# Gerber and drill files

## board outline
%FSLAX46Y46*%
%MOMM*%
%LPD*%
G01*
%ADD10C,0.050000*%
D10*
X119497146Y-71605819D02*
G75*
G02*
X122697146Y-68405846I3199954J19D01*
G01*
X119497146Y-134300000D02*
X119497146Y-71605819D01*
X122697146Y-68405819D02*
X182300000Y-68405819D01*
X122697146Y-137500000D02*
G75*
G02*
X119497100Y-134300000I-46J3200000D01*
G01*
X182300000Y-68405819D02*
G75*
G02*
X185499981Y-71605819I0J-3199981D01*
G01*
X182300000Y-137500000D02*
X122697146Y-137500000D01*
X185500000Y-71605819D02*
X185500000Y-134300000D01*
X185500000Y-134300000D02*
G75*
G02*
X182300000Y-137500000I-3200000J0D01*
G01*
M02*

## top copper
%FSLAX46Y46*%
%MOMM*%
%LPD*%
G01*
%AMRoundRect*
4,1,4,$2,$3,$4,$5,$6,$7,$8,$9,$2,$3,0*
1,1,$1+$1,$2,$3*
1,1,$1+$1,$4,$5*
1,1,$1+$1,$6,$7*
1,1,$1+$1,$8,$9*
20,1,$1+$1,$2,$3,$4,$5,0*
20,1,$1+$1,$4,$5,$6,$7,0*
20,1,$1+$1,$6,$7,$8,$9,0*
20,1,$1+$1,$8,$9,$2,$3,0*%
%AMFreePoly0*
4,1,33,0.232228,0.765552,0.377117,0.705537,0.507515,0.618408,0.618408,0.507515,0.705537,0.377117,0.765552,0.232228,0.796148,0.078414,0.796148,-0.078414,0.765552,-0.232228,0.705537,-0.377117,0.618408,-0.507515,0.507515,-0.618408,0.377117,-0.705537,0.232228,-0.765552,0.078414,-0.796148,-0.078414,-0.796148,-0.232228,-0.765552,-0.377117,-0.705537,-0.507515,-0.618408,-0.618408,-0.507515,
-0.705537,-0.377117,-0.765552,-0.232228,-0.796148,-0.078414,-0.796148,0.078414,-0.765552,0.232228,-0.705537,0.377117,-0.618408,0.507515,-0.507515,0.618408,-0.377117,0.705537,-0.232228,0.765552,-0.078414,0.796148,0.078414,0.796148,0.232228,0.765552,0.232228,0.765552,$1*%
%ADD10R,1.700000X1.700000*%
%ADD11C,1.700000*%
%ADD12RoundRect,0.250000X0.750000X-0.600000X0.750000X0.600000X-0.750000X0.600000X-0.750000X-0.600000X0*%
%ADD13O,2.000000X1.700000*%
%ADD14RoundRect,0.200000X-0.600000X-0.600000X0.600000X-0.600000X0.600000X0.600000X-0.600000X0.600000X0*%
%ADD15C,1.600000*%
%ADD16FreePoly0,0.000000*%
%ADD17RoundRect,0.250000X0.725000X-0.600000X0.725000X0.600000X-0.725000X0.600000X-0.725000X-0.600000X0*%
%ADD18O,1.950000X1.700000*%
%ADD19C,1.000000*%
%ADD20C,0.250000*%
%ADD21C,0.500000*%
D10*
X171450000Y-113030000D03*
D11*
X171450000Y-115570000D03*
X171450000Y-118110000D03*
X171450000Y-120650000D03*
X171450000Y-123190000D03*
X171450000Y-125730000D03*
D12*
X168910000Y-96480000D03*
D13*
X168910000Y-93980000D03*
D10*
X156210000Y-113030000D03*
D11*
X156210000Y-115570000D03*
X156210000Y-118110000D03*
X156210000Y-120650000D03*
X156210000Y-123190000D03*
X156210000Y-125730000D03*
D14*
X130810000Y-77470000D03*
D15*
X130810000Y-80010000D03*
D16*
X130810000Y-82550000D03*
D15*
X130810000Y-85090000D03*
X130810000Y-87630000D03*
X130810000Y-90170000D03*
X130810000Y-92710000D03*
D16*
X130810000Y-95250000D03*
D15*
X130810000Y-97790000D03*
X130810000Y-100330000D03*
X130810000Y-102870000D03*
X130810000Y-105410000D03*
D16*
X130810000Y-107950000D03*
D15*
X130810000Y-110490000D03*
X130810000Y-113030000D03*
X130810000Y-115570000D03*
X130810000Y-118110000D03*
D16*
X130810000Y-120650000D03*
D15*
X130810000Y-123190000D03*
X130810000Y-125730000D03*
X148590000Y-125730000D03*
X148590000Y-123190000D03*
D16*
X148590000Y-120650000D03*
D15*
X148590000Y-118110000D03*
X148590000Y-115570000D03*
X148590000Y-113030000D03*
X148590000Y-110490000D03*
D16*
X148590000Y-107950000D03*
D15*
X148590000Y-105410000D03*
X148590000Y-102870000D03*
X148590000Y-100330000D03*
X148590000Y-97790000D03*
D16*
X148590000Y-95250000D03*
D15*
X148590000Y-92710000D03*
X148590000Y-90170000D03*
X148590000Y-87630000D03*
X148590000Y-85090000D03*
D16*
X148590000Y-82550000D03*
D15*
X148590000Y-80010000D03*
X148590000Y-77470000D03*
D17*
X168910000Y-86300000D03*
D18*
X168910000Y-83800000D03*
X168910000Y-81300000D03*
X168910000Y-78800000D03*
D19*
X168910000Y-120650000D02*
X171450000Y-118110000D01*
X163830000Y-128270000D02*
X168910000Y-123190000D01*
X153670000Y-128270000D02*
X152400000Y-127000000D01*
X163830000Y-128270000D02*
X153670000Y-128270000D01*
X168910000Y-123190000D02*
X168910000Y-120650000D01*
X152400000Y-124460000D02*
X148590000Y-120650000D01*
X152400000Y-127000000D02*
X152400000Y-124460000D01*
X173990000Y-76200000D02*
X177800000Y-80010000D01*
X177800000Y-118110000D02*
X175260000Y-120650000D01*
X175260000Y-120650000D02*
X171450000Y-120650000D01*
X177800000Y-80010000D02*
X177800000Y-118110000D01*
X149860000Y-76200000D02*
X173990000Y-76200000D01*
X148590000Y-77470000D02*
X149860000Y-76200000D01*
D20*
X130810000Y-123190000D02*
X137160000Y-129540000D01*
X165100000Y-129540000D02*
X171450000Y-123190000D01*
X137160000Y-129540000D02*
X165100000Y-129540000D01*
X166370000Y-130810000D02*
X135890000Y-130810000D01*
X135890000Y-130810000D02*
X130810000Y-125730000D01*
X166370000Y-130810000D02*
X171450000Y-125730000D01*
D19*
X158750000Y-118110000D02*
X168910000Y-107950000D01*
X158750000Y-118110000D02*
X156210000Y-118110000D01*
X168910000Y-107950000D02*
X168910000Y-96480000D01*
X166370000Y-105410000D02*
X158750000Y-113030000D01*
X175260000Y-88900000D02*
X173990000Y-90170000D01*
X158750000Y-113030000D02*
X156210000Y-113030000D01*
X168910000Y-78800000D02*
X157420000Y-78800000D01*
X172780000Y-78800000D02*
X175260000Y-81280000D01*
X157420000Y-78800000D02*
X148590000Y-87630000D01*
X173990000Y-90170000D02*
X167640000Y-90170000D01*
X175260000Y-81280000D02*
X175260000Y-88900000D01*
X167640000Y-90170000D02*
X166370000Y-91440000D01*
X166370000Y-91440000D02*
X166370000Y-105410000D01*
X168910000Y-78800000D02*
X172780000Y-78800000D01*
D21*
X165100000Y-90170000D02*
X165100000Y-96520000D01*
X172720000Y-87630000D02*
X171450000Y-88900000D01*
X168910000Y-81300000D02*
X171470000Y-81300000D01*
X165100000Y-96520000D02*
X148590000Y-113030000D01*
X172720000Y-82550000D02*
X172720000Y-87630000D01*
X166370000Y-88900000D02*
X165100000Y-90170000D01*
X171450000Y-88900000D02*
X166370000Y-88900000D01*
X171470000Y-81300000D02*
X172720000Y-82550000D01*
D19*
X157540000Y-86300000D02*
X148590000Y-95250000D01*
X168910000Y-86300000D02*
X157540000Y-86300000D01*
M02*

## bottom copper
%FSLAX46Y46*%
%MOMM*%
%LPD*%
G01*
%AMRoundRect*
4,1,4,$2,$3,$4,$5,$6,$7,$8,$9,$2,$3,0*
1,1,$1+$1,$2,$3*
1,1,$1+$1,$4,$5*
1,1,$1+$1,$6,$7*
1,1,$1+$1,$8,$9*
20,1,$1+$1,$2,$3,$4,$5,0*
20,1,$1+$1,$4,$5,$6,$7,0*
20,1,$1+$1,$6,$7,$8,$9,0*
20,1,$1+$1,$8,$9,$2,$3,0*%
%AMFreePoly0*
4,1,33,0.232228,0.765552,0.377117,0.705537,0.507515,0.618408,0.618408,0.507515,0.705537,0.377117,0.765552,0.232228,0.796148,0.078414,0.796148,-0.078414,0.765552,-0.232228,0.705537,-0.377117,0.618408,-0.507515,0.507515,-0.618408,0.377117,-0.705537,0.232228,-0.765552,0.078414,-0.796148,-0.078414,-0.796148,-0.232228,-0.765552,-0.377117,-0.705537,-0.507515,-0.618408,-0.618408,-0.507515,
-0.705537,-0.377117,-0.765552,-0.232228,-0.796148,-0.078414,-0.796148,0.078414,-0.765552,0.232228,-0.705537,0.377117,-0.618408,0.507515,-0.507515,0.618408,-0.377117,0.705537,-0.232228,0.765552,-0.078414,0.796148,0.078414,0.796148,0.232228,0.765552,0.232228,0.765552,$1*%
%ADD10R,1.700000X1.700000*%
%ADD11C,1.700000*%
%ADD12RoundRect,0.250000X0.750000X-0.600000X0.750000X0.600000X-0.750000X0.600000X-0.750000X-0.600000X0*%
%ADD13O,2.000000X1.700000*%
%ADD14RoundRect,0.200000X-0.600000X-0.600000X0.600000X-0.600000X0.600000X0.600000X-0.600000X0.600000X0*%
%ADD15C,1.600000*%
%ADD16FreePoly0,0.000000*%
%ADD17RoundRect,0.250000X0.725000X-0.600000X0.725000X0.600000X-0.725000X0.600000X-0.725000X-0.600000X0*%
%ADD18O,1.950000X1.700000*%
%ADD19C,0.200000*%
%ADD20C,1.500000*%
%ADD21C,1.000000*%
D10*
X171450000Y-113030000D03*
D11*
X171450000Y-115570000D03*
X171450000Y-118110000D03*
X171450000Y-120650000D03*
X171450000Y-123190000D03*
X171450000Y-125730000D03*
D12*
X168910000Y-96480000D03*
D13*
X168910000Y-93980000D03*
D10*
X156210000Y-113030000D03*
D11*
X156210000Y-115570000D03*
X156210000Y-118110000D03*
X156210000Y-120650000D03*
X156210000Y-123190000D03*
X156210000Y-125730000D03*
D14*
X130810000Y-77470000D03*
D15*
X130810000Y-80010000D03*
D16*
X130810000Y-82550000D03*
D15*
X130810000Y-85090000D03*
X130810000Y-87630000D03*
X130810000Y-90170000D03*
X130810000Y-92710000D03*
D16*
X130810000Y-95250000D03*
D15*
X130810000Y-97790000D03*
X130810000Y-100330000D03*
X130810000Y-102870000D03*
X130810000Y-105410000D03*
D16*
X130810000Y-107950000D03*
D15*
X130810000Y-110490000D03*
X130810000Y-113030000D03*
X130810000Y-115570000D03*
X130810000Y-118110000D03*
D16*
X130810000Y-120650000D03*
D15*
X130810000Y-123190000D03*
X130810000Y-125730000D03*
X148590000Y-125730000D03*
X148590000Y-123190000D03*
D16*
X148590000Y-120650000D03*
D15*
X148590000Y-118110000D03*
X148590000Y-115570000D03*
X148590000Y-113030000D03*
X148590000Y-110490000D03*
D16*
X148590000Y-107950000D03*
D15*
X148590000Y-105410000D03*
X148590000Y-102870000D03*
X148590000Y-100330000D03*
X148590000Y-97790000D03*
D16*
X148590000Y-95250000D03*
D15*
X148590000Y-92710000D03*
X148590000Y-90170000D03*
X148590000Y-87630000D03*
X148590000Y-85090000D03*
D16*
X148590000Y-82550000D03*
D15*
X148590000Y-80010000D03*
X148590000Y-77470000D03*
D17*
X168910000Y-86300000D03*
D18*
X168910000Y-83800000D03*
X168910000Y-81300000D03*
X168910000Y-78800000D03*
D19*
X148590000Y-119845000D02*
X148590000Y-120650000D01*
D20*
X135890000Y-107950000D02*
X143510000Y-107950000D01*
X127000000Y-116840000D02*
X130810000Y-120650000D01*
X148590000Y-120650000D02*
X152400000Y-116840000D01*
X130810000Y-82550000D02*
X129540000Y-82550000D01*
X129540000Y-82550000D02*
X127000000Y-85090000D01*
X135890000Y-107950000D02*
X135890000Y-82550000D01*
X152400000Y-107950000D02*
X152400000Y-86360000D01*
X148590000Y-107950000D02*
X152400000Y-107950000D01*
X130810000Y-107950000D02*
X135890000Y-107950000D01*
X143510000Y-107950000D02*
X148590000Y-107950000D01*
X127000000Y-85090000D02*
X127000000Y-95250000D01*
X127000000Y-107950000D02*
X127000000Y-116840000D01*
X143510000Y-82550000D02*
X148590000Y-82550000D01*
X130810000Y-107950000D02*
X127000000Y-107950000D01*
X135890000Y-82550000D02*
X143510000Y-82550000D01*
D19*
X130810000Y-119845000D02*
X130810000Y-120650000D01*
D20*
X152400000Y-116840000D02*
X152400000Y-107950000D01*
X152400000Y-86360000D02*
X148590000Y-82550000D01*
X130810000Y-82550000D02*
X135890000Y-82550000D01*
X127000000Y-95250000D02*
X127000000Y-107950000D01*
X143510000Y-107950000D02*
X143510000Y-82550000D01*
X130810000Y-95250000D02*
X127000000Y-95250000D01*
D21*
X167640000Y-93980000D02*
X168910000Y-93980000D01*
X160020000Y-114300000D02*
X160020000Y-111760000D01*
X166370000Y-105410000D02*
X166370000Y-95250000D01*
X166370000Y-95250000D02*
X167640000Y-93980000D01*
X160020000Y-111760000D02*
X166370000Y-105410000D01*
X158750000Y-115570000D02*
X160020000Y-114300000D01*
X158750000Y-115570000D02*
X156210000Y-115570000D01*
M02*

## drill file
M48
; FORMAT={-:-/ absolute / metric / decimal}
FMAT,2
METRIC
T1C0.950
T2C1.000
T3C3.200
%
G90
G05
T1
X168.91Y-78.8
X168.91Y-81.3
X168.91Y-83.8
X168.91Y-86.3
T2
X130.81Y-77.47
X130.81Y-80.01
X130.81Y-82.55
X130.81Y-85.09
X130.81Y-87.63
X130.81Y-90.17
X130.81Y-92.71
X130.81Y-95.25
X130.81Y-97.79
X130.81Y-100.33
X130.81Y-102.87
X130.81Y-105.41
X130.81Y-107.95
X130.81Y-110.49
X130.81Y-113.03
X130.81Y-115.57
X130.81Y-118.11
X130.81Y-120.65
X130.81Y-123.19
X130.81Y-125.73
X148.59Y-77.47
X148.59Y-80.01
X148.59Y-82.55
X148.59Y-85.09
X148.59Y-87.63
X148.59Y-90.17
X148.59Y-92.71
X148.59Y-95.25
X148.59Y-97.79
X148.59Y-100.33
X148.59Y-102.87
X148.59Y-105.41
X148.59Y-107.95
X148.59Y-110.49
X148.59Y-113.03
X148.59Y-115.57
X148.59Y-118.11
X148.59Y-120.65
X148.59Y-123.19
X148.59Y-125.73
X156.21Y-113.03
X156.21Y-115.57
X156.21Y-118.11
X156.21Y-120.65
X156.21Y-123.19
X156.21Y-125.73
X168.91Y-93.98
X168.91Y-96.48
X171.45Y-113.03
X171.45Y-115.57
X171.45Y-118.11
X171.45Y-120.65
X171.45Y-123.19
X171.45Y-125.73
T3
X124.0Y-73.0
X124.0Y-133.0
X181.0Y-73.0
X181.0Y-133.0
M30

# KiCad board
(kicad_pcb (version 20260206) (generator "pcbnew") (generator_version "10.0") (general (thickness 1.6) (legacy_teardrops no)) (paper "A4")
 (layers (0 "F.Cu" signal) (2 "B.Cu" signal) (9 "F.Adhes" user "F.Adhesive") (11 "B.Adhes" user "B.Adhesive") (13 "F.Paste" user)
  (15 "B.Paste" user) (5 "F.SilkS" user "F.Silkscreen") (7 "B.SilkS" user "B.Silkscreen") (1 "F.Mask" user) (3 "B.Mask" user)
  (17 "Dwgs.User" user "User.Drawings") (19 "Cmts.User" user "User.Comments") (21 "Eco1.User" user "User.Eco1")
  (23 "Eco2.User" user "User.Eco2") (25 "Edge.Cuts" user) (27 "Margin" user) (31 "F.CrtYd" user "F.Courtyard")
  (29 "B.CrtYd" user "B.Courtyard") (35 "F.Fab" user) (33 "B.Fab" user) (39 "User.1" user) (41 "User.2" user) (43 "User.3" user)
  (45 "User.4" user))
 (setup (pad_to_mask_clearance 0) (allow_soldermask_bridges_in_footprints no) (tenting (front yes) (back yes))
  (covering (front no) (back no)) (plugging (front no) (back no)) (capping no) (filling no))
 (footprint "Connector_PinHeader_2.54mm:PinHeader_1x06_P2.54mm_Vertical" (layer "F.Cu") (at 171.45 113.03)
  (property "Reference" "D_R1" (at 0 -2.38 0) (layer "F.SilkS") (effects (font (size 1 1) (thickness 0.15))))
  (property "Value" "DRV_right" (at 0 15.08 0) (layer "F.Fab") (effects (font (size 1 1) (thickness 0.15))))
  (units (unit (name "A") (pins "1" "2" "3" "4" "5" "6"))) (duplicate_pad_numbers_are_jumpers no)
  (pad "1" thru_hole rect (at 0 0) (size 1.7 1.7) (drill 1) (layers "*.Cu" "*.Mask") (remove_unused_layers no) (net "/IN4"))
  (pad "2" thru_hole circle (at 0 2.54) (size 1.7 1.7) (drill 1) (layers "*.Cu" "*.Mask") (remove_unused_layers no) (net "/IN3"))
  (pad "3" thru_hole circle (at 0 5.08) (size 1.7 1.7) (drill 1) (layers "*.Cu" "*.Mask") (remove_unused_layers no) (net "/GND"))
  (pad "4" thru_hole circle (at 0 7.62) (size 1.7 1.7) (drill 1) (layers "*.Cu" "*.Mask") (remove_unused_layers no) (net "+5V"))
  (pad "5" thru_hole circle (at 0 10.16) (size 1.7 1.7) (drill 1) (layers "*.Cu" "*.Mask") (remove_unused_layers no) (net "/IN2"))
  (pad "6" thru_hole circle (at 0 12.7) (size 1.7 1.7) (drill 1) (layers "*.Cu" "*.Mask") (remove_unused_layers no) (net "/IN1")))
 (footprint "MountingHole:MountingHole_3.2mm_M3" (layer "F.Cu") (at 181 133)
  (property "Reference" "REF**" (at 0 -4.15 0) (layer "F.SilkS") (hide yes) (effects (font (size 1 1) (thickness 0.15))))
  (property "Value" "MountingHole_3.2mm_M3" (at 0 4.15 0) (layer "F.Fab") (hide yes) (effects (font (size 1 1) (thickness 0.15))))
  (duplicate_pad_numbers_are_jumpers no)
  (pad "" np_thru_hole circle (at 0 0) (size 3.2 3.2) (drill 3.2) (layers "*.Cu" "*.Mask")))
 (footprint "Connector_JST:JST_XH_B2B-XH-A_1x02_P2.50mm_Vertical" (layer "F.Cu") (at 168.91 96.48 90)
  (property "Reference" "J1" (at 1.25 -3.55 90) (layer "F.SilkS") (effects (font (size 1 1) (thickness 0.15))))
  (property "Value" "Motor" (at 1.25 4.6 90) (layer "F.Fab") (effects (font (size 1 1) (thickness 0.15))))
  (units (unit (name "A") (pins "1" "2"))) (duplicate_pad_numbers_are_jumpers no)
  (pad "1" thru_hole roundrect (at 0 0 90) (size 1.7 2) (drill 1) (layers "*.Cu" "*.Mask") (remove_unused_layers no)
   (roundrect_rratio 0.147059) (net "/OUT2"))
  (pad "2" thru_hole oval (at 2.5 0 90) (size 1.7 2) (drill 1) (layers "*.Cu" "*.Mask") (remove_unused_layers no) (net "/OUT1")))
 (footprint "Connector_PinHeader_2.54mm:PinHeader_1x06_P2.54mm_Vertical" (layer "F.Cu") (at 156.21 113.03)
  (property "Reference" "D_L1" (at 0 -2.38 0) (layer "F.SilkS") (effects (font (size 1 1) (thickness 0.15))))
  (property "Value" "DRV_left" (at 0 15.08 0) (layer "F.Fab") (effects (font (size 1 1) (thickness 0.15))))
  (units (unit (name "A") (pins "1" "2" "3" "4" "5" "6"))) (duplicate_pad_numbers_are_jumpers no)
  (pad "1" thru_hole rect (at 0 0) (size 1.7 1.7) (drill 1) (layers "*.Cu" "*.Mask") (remove_unused_layers no) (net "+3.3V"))
  (pad "2" thru_hole circle (at 0 2.54) (size 1.7 1.7) (drill 1) (layers "*.Cu" "*.Mask") (remove_unused_layers no) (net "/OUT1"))
  (pad "3" thru_hole circle (at 0 5.08) (size 1.7 1.7) (drill 1) (layers "*.Cu" "*.Mask") (remove_unused_layers no) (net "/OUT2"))
  (pad "4" thru_hole circle (at 0 7.62) (size 1.7 1.7) (drill 1) (layers "*.Cu" "*.Mask") (remove_unused_layers no) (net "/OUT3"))
  (pad "5" thru_hole circle (at 0 10.16) (size 1.7 1.7) (drill 1) (layers "*.Cu" "*.Mask") (remove_unused_layers no) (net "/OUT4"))
  (pad "6" thru_hole circle (at 0 12.7) (size 1.7 1.7) (drill 1) (layers "*.Cu" "*.Mask") (remove_unused_layers no) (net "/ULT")))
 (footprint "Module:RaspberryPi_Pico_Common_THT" (layer "F.Cu") (at 130.81 77.47)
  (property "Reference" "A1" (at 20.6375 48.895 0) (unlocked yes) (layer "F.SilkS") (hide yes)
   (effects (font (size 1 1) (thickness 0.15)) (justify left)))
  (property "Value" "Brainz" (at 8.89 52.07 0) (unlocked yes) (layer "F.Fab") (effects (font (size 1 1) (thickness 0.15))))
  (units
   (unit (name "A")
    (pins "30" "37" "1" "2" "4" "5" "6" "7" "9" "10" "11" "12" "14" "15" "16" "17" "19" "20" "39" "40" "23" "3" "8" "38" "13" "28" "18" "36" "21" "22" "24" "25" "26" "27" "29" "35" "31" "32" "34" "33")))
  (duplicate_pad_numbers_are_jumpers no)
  (pad "1" thru_hole roundrect (at 0 0) (size 1.6 1.6) (drill 1) (layers "*.Cu" "*.Mask") (remove_unused_layers no) (roundrect_rratio 0.125)
   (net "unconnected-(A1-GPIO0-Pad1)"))
  (pad "2" thru_hole circle (at 0 2.54) (size 1.6 1.6) (drill 1) (layers "*.Cu" "*.Mask") (remove_unused_layers no)
   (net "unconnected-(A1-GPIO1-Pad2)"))
  (pad "3" thru_hole custom (at 0 5.08) (size 1.6 1.6) (drill 1) (layers "*.Cu" "*.Mask") (remove_unused_layers no) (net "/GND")
   (options (clearance outline) (anchor circle)) (primitives))
  (pad "4" thru_hole circle (at 0 7.62) (size 1.6 1.6) (drill 1) (layers "*.Cu" "*.Mask") (remove_unused_layers no)
   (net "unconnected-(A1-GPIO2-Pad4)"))
  (pad "5" thru_hole circle (at 0 10.16) (size 1.6 1.6) (drill 1) (layers "*.Cu" "*.Mask") (remove_unused_layers no)
   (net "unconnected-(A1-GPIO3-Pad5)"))
  (pad "6" thru_hole circle (at 0 12.7) (size 1.6 1.6) (drill 1) (layers "*.Cu" "*.Mask") (remove_unused_layers no)
   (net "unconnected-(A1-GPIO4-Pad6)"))
  (pad "7" thru_hole circle (at 0 15.24) (size 1.6 1.6) (drill 1) (layers "*.Cu" "*.Mask") (remove_unused_layers no)
   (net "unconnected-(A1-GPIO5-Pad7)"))
  (pad "8" thru_hole custom (at 0 17.78) (size 1.6 1.6) (drill 1) (layers "*.Cu" "*.Mask") (remove_unused_layers no) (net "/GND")
   (options (clearance outline) (anchor circle)) (primitives))
  (pad "9" thru_hole circle (at 0 20.32) (size 1.6 1.6) (drill 1) (layers "*.Cu" "*.Mask") (remove_unused_layers no)
   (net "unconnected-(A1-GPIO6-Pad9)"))
  (pad "10" thru_hole circle (at 0 22.86) (size 1.6 1.6) (drill 1) (layers "*.Cu" "*.Mask") (remove_unused_layers no)
   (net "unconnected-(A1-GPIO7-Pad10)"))
  (pad "11" thru_hole circle (at 0 25.4) (size 1.6 1.6) (drill 1) (layers "*.Cu" "*.Mask") (remove_unused_layers no)
   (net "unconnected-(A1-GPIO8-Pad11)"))
  (pad "12" thru_hole circle (at 0 27.94) (size 1.6 1.6) (drill 1) (layers "*.Cu" "*.Mask") (remove_unused_layers no)
   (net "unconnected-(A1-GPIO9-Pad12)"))
  (pad "13" thru_hole custom (at 0 30.48) (size 1.6 1.6) (drill 1) (layers "*.Cu" "*.Mask") (remove_unused_layers no) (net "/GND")
   (options (clearance outline) (anchor circle)) (primitives))
  (pad "14" thru_hole circle (at 0 33.02) (size 1.6 1.6) (drill 1) (layers "*.Cu" "*.Mask") (remove_unused_layers no)
   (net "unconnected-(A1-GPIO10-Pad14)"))
  (pad "15" thru_hole circle (at 0 35.56) (size 1.6 1.6) (drill 1) (layers "*.Cu" "*.Mask") (remove_unused_layers no)
   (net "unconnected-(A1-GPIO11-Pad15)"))
  (pad "16" thru_hole circle (at 0 38.1) (size 1.6 1.6) (drill 1) (layers "*.Cu" "*.Mask") (remove_unused_layers no)
   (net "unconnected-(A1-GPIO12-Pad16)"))
  (pad "17" thru_hole circle (at 0 40.64) (size 1.6 1.6) (drill 1) (layers "*.Cu" "*.Mask") (remove_unused_layers no)
   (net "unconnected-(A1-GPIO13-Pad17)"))
  (pad "18" thru_hole custom (at 0 43.18) (size 1.6 1.6) (drill 1) (layers "*.Cu" "*.Mask") (remove_unused_layers no) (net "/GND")
   (options (clearance outline) (anchor circle)) (primitives))
  (pad "19" thru_hole circle (at 0 45.72) (size 1.6 1.6) (drill 1) (layers "*.Cu" "*.Mask") (remove_unused_layers no) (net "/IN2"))
  (pad "20" thru_hole circle (at 0 48.26) (size 1.6 1.6) (drill 1) (layers "*.Cu" "*.Mask") (remove_unused_layers no) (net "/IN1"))
  (pad "21" thru_hole circle (at 17.78 48.26) (size 1.6 1.6) (drill 1) (layers "*.Cu" "*.Mask") (remove_unused_layers no)
   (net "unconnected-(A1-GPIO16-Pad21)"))
  (pad "22" thru_hole circle (at 17.78 45.72) (size 1.6 1.6) (drill 1) (layers "*.Cu" "*.Mask") (remove_unused_layers no)
   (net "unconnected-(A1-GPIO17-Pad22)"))
  (pad "23" thru_hole custom (at 17.78 43.18) (size 1.6 1.6) (drill 1) (layers "*.Cu" "*.Mask") (remove_unused_layers no) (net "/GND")
   (options (clearance outline) (anchor circle)) (primitives))
  (pad "24" thru_hole circle (at 17.78 40.64) (size 1.6 1.6) (drill 1) (layers "*.Cu" "*.Mask") (remove_unused_layers no)
   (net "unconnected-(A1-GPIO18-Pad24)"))
  (pad "25" thru_hole circle (at 17.78 38.1) (size 1.6 1.6) (drill 1) (layers "*.Cu" "*.Mask") (remove_unused_layers no)
   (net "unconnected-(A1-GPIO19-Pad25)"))
  (pad "26" thru_hole circle (at 17.78 35.56) (size 1.6 1.6) (drill 1) (layers "*.Cu" "*.Mask") (remove_unused_layers no)
   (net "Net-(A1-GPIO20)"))
  (pad "27" thru_hole circle (at 17.78 33.02) (size 1.6 1.6) (drill 1) (layers "*.Cu" "*.Mask") (remove_unused_layers no)
   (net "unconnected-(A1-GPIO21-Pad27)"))
  (pad "28" thru_hole custom (at 17.78 30.48) (size 1.6 1.6) (drill 1) (layers "*.Cu" "*.Mask") (remove_unused_layers no) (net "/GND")
   (options (clearance outline) (anchor circle)) (primitives))
  (pad "29" thru_hole circle (at 17.78 27.94) (size 1.6 1.6) (drill 1) (layers "*.Cu" "*.Mask") (remove_unused_layers no)
   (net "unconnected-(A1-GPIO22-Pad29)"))
  (pad "30" thru_hole circle (at 17.78 25.4) (size 1.6 1.6) (drill 1) (layers "*.Cu" "*.Mask") (remove_unused_layers no)
   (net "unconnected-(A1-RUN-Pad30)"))
  (pad "31" thru_hole circle (at 17.78 22.86) (size 1.6 1.6) (drill 1) (layers "*.Cu" "*.Mask") (remove_unused_layers no)
   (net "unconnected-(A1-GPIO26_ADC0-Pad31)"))
  (pad "32" thru_hole circle (at 17.78 20.32) (size 1.6 1.6) (drill 1) (layers "*.Cu" "*.Mask") (remove_unused_layers no)
   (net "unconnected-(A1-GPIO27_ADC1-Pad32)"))
  (pad "33" thru_hole custom (at 17.78 17.78) (size 1.6 1.6) (drill 1) (layers "*.Cu" "*.Mask") (remove_unused_layers no)
   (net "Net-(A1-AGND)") (options (clearance outline) (anchor circle)) (primitives))
  (pad "34" thru_hole circle (at 17.78 15.24) (size 1.6 1.6) (drill 1) (layers "*.Cu" "*.Mask") (remove_unused_layers no)
   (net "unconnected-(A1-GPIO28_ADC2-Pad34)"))
  (pad "35" thru_hole circle (at 17.78 12.7) (size 1.6 1.6) (drill 1) (layers "*.Cu" "*.Mask") (remove_unused_layers no)
   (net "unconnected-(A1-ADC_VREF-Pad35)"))
  (pad "36" thru_hole circle (at 17.78 10.16) (size 1.6 1.6) (drill 1) (layers "*.Cu" "*.Mask") (remove_unused_layers no) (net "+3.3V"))
  (pad "37" thru_hole circle (at 17.78 7.62) (size 1.6 1.6) (drill 1) (layers "*.Cu" "*.Mask") (remove_unused_layers no)
   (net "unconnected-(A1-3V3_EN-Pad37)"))
  (pad "38" thru_hole custom (at 17.78 5.08) (size 1.6 1.6) (drill 1) (layers "*.Cu" "*.Mask") (remove_unused_layers no) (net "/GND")
   (options (clearance outline) (anchor circle)) (primitives))
  (pad "39" thru_hole circle (at 17.78 2.54) (size 1.6 1.6) (drill 1) (layers "*.Cu" "*.Mask") (remove_unused_layers no)
   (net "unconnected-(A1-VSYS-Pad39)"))
  (pad "40" thru_hole circle (at 17.78 0) (size 1.6 1.6) (drill 1) (layers "*.Cu" "*.Mask") (remove_unused_layers no) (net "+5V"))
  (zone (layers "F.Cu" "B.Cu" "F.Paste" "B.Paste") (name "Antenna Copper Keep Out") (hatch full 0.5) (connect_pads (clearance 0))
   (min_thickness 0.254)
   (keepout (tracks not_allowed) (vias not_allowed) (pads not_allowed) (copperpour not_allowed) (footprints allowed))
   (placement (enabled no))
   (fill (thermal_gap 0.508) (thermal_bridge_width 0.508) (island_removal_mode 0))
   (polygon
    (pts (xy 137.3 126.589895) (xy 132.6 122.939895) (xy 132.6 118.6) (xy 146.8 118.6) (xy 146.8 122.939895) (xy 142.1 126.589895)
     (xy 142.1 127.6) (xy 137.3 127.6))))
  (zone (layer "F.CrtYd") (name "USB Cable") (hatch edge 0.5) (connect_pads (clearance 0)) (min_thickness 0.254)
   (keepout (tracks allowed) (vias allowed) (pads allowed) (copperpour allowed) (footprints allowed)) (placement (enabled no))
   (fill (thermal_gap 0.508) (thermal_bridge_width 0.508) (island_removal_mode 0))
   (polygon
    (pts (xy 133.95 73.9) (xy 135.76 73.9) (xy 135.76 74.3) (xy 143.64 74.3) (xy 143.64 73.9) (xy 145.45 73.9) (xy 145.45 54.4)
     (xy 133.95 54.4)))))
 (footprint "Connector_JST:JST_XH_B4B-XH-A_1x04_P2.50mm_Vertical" (layer "F.Cu") (at 168.91 86.3 90)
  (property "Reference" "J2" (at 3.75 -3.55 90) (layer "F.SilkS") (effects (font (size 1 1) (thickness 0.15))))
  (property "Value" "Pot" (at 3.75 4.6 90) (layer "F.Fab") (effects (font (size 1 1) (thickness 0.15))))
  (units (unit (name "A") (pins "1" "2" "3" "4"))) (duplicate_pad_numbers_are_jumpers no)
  (pad "1" thru_hole roundrect (at 0 0 90) (size 1.7 1.95) (drill 0.95) (layers "*.Cu" "*.Mask") (remove_unused_layers no)
   (roundrect_rratio 0.147059) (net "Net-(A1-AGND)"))
  (pad "2" thru_hole oval (at 2.5 0 90) (size 1.7 1.95) (drill 0.95) (layers "*.Cu" "*.Mask") (remove_unused_layers no)
   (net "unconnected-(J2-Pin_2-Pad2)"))
  (pad "3" thru_hole oval (at 5 0 90) (size 1.7 1.95) (drill 0.95) (layers "*.Cu" "*.Mask") (remove_unused_layers no)
   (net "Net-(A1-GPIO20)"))
  (pad "4" thru_hole oval (at 7.5 0 90) (size 1.7 1.95) (drill 0.95) (layers "*.Cu" "*.Mask") (remove_unused_layers no) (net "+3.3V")))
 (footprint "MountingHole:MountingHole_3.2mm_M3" (layer "F.Cu") (at 124 133)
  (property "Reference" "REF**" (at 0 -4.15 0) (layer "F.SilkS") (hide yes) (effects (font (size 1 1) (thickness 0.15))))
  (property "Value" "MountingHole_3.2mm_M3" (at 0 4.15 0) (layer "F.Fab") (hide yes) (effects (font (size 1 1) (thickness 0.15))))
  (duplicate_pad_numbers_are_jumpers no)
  (pad "" np_thru_hole circle (at 0 0) (size 3.2 3.2) (drill 3.2) (layers "*.Cu" "*.Mask")))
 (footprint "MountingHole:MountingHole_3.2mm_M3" (layer "F.Cu") (at 124 73)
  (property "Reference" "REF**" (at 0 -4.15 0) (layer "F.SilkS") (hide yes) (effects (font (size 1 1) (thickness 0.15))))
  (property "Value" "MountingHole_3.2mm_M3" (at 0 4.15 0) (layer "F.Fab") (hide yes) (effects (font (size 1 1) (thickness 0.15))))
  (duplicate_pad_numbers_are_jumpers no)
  (pad "" np_thru_hole circle (at 0 0) (size 3.2 3.2) (drill 3.2) (layers "*.Cu" "*.Mask")))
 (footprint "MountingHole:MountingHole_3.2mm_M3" (layer "F.Cu") (at 181 73)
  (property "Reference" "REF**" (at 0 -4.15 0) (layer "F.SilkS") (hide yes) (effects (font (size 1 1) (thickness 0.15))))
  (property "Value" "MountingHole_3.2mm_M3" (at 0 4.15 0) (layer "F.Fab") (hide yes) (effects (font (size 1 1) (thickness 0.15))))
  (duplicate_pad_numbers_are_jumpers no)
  (pad "" np_thru_hole circle (at 0 0) (size 3.2 3.2) (drill 3.2) (layers "*.Cu" "*.Mask")))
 (gr_arc (start 119.497146 71.605819) (mid 120.434404 69.343077) (end 122.697146 68.405819) (stroke (width 0.05) (type default))
  (layer "Edge.Cuts"))
 (gr_line (start 119.497146 134.3) (end 119.497146 71.605819) (stroke (width 0.05) (type default)) (layer "Edge.Cuts"))
 (gr_line (start 122.697146 68.405819) (end 182.3 68.405819) (stroke (width 0.05) (type default)) (layer "Edge.Cuts"))
 (gr_arc (start 122.697146 137.5) (mid 120.434404 136.562742) (end 119.497146 134.3) (stroke (width 0.05) (type default))
  (layer "Edge.Cuts"))
 (gr_arc (start 182.3 68.405819) (mid 184.562735 69.343078) (end 185.5 71.605819) (stroke (width 0.05) (type default)) (layer "Edge.Cuts"))
 (gr_line (start 182.3 137.5) (end 122.697146 137.5) (stroke (width 0.05) (type default)) (layer "Edge.Cuts"))
 (gr_line (start 185.5 71.605819) (end 185.5 134.3) (stroke (width 0.05) (type default)) (layer "Edge.Cuts"))
 (gr_arc (start 185.5 134.3) (mid 184.562742 136.562742) (end 182.3 137.5) (stroke (width 0.05) (type default)) (layer "Edge.Cuts"))
 (segment (start 168.91 120.65) (end 171.45 118.11) (width 1) (layer "F.Cu") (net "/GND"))
 (segment (start 163.83 128.27) (end 168.91 123.19) (width 1) (layer "F.Cu") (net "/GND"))
 (segment (start 153.67 128.27) (end 152.4 127) (width 1) (layer "F.Cu") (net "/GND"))
 (segment (start 163.83 128.27) (end 153.67 128.27) (width 1) (layer "F.Cu") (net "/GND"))
 (segment (start 168.91 123.19) (end 168.91 120.65) (width 1) (layer "F.Cu") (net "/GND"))
 (segment (start 152.4 124.46) (end 148.59 120.65) (width 1) (layer "F.Cu") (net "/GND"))
 (segment (start 152.4 127) (end 152.4 124.46) (width 1) (layer "F.Cu") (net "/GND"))
 (segment (start 148.59 119.845) (end 148.59 120.65) (width 0.2) (layer "B.Cu") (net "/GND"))
 (segment (start 135.89 107.95) (end 143.51 107.95) (width 1.5) (layer "B.Cu") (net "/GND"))
 (segment (start 127 116.84) (end 130.81 120.65) (width 1.5) (layer "B.Cu") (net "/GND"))
 (segment (start 148.59 120.65) (end 152.4 116.84) (width 1.5) (layer "B.Cu") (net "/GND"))
 (segment (start 130.81 82.55) (end 129.54 82.55) (width 1.5) (layer "B.Cu") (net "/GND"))
 (segment (start 129.54 82.55) (end 127 85.09) (width 1.5) (layer "B.Cu") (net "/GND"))
 (segment (start 135.89 107.95) (end 135.89 82.55) (width 1.5) (layer "B.Cu") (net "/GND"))
 (segment (start 152.4 107.95) (end 152.4 86.36) (width 1.5) (layer "B.Cu") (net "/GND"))
 (segment (start 148.59 107.95) (end 152.4 107.95) (width 1.5) (layer "B.Cu") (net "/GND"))
 (segment (start 130.81 107.95) (end 135.89 107.95) (width 1.5) (layer "B.Cu") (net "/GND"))
 (segment (start 143.51 107.95) (end 148.59 107.95) (width 1.5) (layer "B.Cu") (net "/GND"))
 (segment (start 127 85.09) (end 127 95.25) (width 1.5) (layer "B.Cu") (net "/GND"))
 (segment (start 127 107.95) (end 127 116.84) (width 1.5) (layer "B.Cu") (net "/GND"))
 (segment (start 143.51 82.55) (end 148.59 82.55) (width 1.5) (layer "B.Cu") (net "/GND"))
 (segment (start 130.81 107.95) (end 127 107.95) (width 1.5) (layer "B.Cu") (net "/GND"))
 (segment (start 135.89 82.55) (end 143.51 82.55) (width 1.5) (layer "B.Cu") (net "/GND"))
 (segment (start 130.81 119.845) (end 130.81 120.65) (width 0.2) (layer "B.Cu") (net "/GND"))
 (segment (start 152.4 116.84) (end 152.4 107.95) (width 1.5) (layer "B.Cu") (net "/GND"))
 (segment (start 152.4 86.36) (end 148.59 82.55) (width 1.5) (layer "B.Cu") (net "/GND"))
 (segment (start 130.81 82.55) (end 135.89 82.55) (width 1.5) (layer "B.Cu") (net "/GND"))
 (segment (start 127 95.25) (end 127 107.95) (width 1.5) (layer "B.Cu") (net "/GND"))
 (segment (start 143.51 107.95) (end 143.51 82.55) (width 1.5) (layer "B.Cu") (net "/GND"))
 (segment (start 130.81 95.25) (end 127 95.25) (width 1.5) (layer "B.Cu") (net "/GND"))
 (segment (start 173.99 76.2) (end 177.8 80.01) (width 1) (layer "F.Cu") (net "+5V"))
 (segment (start 177.8 118.11) (end 175.26 120.65) (width 1) (layer "F.Cu") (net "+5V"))
 (segment (start 175.26 120.65) (end 171.45 120.65) (width 1) (layer "F.Cu") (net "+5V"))
 (segment (start 177.8 80.01) (end 177.8 118.11) (width 1) (layer "F.Cu") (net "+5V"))
 (segment (start 149.86 76.2) (end 173.99 76.2) (width 1) (layer "F.Cu") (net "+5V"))
 (segment (start 148.59 77.47) (end 149.86 76.2) (width 1) (layer "F.Cu") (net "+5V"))
 (segment (start 130.81 123.19) (end 137.16 129.54) (width 0.25) (layer "F.Cu") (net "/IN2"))
 (segment (start 165.1 129.54) (end 171.45 123.19) (width 0.25) (layer "F.Cu") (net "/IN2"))
 (segment (start 137.16 129.54) (end 165.1 129.54) (width 0.25) (layer "F.Cu") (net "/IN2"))
 (segment (start 166.37 130.81) (end 135.89 130.81) (width 0.25) (layer "F.Cu") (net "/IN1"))
 (segment (start 135.89 130.81) (end 130.81 125.73) (width 0.25) (layer "F.Cu") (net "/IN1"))
 (segment (start 166.37 130.81) (end 171.45 125.73) (width 0.25) (layer "F.Cu") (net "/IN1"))
 (segment (start 158.75 118.11) (end 168.91 107.95) (width 1) (layer "F.Cu") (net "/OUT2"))
 (segment (start 158.75 118.11) (end 156.21 118.11) (width 1) (layer "F.Cu") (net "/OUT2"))
 (segment (start 168.91 107.95) (end 168.91 96.48) (width 1) (layer "F.Cu") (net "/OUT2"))
 (segment (start 167.64 93.98) (end 168.91 93.98) (width 1) (layer "B.Cu") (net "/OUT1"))
 (segment (start 160.02 114.3) (end 160.02 111.76) (width 1) (layer "B.Cu") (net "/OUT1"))
 (segment (start 166.37 105.41) (end 166.37 95.25) (width 1) (layer "B.Cu") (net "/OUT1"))
 (segment (start 166.37 95.25) (end 167.64 93.98) (width 1) (layer "B.Cu") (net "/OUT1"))
 (segment (start 160.02 111.76) (end 166.37 105.41) (width 1) (layer "B.Cu") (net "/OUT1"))
 (segment (start 158.75 115.57) (end 160.02 114.3) (width 1) (layer "B.Cu") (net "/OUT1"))
 (segment (start 158.75 115.57) (end 156.21 115.57) (width 1) (layer "B.Cu") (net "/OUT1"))
 (segment (start 166.37 105.41) (end 158.75 113.03) (width 1) (layer "F.Cu") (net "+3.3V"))
 (segment (start 175.26 88.9) (end 173.99 90.17) (width 1) (layer "F.Cu") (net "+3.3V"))
 (segment (start 158.75 113.03) (end 156.21 113.03) (width 1) (layer "F.Cu") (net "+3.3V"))
 (segment (start 168.91 78.8) (end 157.42 78.8) (width 1) (layer "F.Cu") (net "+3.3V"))
 (segment (start 172.78 78.8) (end 175.26 81.28) (width 1) (layer "F.Cu") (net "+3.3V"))
 (segment (start 157.42 78.8) (end 148.59 87.63) (width 1) (layer "F.Cu") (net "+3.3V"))
 (segment (start 173.99 90.17) (end 167.64 90.17) (width 1) (layer "F.Cu") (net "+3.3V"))
 (segment (start 175.26 81.28) (end 175.26 88.9) (width 1) (layer "F.Cu") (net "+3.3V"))
 (segment (start 167.64 90.17) (end 166.37 91.44) (width 1) (layer "F.Cu") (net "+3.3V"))
 (segment (start 166.37 91.44) (end 166.37 105.41) (width 1) (layer "F.Cu") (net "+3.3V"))
 (segment (start 168.91 78.8) (end 172.78 78.8) (width 1) (layer "F.Cu") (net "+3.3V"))
 (segment (start 165.1 90.17) (end 165.1 96.52) (width 0.5) (layer "F.Cu") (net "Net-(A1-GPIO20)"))
 (segment (start 172.72 87.63) (end 171.45 88.9) (width 0.5) (layer "F.Cu") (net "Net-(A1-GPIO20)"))
 (segment (start 168.91 81.3) (end 171.47 81.3) (width 0.5) (layer "F.Cu") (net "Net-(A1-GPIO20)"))
 (segment (start 165.1 96.52) (end 148.59 113.03) (width 0.5) (layer "F.Cu") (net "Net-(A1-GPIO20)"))
 (segment (start 172.72 82.55) (end 172.72 87.63) (width 0.5) (layer "F.Cu") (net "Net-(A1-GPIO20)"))
 (segment (start 166.37 88.9) (end 165.1 90.17) (width 0.5) (layer "F.Cu") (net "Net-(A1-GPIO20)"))
 (segment (start 171.45 88.9) (end 166.37 88.9) (width 0.5) (layer "F.Cu") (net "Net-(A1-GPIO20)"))
 (segment (start 171.47 81.3) (end 172.72 82.55) (width 0.5) (layer "F.Cu") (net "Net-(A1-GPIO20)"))
 (segment (start 157.54 86.3) (end 148.59 95.25) (width 1) (layer "F.Cu") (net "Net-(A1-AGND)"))
 (segment (start 168.91 86.3) (end 157.54 86.3) (width 1) (layer "F.Cu") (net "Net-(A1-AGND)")))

